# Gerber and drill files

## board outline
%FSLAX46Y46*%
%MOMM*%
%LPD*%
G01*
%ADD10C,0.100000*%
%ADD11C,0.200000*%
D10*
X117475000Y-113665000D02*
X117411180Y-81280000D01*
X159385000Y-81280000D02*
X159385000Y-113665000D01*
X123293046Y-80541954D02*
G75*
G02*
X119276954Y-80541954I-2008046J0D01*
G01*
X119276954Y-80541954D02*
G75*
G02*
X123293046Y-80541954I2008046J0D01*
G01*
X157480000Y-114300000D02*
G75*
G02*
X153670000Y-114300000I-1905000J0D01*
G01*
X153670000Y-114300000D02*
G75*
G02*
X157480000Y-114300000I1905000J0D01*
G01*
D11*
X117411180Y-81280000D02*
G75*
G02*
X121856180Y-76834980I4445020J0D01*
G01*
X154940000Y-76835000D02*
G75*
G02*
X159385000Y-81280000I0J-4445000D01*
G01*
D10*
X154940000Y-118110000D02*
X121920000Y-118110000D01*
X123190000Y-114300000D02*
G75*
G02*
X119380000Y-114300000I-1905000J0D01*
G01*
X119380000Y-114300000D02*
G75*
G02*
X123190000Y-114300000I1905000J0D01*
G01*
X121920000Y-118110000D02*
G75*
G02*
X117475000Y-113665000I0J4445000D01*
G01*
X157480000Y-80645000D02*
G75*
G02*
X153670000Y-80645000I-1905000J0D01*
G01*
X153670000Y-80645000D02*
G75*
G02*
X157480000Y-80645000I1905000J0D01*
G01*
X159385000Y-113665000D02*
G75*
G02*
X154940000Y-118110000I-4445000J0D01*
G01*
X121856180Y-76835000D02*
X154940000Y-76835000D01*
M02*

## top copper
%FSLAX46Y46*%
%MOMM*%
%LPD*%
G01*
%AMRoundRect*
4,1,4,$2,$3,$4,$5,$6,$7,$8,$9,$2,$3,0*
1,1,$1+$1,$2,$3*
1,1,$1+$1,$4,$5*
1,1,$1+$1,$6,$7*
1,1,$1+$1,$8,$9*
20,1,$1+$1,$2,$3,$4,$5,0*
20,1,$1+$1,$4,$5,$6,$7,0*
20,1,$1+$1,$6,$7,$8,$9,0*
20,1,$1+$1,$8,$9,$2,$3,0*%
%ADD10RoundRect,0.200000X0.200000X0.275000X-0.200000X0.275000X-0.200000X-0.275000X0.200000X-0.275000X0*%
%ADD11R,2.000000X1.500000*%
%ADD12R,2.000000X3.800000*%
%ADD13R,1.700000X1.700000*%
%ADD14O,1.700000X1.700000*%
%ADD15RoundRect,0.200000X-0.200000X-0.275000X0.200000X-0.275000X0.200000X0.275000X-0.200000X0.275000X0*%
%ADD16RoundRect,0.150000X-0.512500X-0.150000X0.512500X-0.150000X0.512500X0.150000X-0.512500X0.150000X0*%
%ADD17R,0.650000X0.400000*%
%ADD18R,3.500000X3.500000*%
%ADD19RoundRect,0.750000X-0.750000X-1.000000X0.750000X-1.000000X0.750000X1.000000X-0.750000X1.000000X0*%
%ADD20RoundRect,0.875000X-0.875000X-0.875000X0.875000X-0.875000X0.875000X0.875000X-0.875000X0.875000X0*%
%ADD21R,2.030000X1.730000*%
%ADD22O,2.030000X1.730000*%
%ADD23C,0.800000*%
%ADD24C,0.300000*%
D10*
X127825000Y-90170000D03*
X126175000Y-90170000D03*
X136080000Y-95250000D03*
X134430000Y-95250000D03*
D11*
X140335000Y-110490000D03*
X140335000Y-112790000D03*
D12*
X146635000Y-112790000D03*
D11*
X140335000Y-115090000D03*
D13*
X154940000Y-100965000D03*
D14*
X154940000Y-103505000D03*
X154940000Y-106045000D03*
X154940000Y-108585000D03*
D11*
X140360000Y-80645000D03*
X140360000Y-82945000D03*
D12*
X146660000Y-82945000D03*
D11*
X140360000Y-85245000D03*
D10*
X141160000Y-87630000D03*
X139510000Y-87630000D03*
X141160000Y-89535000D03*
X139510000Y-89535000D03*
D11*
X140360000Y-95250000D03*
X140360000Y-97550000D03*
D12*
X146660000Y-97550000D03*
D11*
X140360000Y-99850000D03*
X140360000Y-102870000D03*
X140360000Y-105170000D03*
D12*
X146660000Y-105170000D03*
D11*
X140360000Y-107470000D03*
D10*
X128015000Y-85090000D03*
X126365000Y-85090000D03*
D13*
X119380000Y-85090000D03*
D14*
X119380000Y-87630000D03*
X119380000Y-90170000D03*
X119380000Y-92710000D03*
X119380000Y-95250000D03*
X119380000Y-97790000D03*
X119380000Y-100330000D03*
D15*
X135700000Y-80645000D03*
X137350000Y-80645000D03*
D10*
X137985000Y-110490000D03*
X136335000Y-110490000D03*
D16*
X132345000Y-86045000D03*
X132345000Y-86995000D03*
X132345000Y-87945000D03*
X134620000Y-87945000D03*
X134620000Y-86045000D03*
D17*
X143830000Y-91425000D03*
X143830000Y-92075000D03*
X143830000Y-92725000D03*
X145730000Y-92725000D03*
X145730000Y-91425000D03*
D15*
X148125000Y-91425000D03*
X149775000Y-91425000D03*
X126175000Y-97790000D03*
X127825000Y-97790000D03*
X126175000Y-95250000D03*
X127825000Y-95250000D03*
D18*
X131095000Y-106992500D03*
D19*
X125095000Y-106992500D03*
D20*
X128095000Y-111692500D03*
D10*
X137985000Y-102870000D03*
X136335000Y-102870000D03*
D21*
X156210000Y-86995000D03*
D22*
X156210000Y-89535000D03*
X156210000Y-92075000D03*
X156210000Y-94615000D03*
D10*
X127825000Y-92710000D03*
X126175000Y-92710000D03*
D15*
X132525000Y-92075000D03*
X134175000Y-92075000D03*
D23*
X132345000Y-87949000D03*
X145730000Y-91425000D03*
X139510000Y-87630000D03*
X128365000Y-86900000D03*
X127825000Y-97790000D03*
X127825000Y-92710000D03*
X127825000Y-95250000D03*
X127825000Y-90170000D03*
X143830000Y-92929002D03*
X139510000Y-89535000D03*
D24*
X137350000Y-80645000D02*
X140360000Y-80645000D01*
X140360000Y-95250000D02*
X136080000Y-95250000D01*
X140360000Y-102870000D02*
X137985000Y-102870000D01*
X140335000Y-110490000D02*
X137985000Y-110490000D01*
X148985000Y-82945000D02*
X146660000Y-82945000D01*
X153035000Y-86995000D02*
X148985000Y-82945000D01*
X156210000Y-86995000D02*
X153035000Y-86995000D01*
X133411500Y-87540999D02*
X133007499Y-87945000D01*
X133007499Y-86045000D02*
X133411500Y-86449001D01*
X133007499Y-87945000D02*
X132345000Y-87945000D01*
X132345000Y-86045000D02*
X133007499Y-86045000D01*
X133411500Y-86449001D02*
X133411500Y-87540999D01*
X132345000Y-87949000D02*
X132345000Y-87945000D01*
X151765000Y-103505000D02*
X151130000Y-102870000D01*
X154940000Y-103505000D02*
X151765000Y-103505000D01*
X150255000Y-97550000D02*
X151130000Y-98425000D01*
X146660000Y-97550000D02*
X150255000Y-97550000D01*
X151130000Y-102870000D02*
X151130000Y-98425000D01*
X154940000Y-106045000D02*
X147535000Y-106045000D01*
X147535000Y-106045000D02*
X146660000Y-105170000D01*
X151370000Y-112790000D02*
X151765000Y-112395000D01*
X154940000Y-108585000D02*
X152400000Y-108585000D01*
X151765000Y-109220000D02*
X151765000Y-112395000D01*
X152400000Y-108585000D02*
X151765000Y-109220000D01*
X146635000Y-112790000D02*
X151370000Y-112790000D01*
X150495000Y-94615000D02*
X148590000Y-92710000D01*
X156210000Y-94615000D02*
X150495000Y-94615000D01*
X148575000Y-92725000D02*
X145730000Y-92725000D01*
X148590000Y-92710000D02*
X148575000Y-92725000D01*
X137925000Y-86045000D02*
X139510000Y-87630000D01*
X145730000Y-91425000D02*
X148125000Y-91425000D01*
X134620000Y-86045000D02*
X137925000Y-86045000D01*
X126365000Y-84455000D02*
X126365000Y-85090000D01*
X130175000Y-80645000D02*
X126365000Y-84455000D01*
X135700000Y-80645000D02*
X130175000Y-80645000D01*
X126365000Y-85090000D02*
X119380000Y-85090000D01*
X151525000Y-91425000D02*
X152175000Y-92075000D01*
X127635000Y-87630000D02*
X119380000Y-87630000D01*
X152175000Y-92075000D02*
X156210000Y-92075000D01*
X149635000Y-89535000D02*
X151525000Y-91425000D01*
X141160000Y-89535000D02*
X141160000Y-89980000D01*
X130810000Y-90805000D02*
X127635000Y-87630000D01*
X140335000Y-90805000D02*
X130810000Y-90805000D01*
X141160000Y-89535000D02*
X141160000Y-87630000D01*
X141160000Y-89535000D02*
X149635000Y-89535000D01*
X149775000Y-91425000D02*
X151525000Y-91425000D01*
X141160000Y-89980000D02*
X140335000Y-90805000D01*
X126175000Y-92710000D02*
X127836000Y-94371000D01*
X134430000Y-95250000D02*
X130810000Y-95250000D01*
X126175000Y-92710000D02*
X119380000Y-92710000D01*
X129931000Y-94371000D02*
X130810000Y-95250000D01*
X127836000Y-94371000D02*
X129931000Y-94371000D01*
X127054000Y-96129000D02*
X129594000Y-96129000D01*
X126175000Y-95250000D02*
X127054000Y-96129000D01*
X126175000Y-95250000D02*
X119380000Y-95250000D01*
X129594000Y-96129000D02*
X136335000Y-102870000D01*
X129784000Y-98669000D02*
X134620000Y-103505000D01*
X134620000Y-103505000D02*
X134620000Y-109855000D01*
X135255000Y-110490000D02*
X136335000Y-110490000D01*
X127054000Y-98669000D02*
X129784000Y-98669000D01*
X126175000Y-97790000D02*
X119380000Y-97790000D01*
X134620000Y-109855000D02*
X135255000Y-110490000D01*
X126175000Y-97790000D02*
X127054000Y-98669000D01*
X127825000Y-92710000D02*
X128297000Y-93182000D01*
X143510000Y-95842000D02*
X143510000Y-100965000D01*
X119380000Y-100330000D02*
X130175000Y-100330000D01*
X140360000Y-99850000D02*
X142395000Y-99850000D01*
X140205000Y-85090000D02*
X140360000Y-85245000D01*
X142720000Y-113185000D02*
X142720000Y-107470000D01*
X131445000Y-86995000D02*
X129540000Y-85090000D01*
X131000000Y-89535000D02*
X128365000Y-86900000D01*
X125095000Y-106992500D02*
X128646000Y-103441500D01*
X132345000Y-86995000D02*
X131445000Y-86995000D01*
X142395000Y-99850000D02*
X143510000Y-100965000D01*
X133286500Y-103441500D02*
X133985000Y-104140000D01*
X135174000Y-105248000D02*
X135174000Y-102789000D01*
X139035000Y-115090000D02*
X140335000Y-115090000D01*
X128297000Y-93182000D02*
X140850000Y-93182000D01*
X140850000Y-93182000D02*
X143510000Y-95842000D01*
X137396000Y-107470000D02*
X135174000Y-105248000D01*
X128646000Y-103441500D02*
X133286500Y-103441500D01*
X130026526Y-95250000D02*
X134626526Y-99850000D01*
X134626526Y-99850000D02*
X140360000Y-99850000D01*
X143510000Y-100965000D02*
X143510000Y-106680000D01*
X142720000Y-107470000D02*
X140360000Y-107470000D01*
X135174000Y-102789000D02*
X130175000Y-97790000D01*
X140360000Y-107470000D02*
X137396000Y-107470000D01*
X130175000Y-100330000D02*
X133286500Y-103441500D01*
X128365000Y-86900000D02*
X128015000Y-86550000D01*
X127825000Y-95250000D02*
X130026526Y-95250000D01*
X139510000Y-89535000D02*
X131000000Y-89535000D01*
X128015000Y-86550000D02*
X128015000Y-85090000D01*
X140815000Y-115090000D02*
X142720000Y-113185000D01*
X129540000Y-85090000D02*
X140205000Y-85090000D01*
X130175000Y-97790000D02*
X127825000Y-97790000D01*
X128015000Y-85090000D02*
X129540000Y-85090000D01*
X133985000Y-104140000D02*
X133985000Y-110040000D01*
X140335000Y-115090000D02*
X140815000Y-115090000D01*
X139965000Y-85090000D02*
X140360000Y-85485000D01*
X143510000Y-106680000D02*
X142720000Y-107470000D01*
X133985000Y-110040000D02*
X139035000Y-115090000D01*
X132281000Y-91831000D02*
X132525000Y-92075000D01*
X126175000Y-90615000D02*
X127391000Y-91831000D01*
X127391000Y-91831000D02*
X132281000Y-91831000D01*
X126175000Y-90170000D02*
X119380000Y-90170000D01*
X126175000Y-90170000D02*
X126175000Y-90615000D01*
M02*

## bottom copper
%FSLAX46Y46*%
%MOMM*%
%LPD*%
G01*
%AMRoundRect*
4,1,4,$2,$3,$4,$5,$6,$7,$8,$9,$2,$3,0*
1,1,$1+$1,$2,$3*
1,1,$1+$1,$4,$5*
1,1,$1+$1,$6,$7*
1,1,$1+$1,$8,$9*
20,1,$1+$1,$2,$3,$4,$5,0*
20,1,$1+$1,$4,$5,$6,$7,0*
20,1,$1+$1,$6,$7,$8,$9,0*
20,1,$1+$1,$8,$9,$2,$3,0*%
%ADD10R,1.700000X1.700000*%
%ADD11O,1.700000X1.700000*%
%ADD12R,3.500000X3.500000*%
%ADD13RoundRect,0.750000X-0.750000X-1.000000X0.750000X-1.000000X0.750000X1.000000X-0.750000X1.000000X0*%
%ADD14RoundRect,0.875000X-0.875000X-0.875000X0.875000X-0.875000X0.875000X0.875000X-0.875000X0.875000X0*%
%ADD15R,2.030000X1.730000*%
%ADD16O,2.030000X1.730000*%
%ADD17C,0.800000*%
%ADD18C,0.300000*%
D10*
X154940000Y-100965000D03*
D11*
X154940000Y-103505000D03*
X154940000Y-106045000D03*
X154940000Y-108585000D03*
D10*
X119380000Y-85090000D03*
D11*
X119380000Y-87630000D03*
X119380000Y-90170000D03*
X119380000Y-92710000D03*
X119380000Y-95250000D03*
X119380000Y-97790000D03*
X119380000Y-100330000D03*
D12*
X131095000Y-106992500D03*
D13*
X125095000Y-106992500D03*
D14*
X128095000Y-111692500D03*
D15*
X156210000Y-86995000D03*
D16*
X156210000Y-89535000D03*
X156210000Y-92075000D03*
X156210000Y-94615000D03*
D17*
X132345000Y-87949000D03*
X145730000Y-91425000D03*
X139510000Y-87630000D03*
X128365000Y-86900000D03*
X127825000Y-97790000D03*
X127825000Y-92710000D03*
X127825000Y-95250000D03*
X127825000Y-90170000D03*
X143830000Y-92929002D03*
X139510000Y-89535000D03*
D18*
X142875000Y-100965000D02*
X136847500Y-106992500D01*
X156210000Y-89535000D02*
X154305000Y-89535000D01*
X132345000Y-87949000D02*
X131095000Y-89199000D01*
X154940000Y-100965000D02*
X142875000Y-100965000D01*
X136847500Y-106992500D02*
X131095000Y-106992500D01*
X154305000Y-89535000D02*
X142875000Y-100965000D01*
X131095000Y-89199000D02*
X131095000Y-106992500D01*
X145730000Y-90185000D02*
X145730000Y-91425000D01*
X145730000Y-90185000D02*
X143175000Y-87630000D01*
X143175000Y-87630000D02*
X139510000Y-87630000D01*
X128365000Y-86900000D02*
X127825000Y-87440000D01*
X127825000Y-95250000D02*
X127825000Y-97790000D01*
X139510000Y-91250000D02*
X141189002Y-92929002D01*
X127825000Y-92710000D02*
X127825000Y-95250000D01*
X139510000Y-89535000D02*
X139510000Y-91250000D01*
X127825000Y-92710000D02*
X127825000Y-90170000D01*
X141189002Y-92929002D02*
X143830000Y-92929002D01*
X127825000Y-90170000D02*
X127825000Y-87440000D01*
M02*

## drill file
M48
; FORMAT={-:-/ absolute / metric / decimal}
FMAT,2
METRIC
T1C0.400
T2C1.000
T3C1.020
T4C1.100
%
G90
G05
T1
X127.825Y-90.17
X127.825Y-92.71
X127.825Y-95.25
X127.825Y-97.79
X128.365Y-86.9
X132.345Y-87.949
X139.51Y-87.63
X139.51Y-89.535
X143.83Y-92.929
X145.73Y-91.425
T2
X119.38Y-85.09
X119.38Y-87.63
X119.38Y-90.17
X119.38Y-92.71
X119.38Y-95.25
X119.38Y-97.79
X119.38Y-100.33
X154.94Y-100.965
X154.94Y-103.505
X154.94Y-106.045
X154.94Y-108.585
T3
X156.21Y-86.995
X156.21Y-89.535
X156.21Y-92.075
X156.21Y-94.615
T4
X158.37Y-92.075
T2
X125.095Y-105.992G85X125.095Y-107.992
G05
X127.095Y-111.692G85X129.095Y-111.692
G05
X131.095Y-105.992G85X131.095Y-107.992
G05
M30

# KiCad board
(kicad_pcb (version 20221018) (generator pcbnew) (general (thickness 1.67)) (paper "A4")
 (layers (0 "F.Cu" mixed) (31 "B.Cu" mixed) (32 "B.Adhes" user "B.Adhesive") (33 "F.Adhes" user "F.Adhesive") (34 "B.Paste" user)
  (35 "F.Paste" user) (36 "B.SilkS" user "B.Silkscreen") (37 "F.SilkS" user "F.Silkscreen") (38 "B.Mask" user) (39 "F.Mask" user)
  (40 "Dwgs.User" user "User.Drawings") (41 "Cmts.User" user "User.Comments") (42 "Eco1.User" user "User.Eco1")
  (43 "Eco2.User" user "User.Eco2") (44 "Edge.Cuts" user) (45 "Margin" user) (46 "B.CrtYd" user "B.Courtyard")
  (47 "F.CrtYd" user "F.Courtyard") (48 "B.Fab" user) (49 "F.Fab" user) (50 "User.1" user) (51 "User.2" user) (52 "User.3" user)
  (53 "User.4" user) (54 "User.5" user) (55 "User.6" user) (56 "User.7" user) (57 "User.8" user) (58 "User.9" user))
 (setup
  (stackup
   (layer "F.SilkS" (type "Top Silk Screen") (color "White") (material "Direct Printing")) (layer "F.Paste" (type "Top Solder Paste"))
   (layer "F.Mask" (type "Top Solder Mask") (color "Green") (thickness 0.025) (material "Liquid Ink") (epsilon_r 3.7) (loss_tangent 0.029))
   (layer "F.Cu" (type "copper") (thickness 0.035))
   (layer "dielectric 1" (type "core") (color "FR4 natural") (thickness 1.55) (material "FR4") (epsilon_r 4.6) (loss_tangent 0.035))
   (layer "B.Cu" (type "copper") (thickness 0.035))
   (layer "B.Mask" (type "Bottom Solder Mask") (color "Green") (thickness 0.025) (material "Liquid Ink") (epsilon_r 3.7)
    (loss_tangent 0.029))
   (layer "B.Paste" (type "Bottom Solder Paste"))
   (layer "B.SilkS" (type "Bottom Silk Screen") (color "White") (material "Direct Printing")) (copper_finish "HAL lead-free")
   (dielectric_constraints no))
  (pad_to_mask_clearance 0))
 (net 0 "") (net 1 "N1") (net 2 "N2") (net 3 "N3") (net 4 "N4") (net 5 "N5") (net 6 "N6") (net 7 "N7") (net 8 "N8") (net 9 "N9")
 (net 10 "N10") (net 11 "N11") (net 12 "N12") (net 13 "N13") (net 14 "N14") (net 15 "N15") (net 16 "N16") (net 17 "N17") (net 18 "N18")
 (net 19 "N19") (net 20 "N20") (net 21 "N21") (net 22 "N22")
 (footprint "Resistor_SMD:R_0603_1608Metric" (layer "F.Cu") (at 127 90.17 180)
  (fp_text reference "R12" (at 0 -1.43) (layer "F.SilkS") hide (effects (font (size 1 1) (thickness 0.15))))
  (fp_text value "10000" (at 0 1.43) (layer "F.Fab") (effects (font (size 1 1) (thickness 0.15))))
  (pad "1" smd roundrect (at -0.825 0 180) (size 0.8 0.95) (layers "F.Cu" "F.Paste" "F.Mask") (roundrect_rratio 0.25) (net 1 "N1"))
  (pad "2" smd roundrect (at 0.825 0 180) (size 0.8 0.95) (layers "F.Cu" "F.Paste" "F.Mask") (roundrect_rratio 0.25) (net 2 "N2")))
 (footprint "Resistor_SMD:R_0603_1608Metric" (layer "F.Cu") (at 135.255 95.25 180)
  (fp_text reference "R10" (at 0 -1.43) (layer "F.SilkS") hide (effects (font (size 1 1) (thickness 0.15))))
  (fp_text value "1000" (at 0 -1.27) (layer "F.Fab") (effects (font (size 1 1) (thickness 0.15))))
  (pad "1" smd roundrect (at -0.825 0 180) (size 0.8 0.95) (layers "F.Cu" "F.Paste" "F.Mask") (roundrect_rratio 0.25) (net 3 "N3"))
  (pad "2" smd roundrect (at 0.825 0 180) (size 0.8 0.95) (layers "F.Cu" "F.Paste" "F.Mask") (roundrect_rratio 0.25) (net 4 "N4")))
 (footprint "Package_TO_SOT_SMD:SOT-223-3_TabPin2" (layer "F.Cu") (at 143.485 112.79)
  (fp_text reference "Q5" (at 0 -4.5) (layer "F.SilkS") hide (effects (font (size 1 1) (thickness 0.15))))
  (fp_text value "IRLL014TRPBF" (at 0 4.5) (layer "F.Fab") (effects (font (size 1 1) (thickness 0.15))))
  (pad "1" smd rect (at -3.15 -2.3) (size 2 1.5) (layers "F.Cu" "F.Paste" "F.Mask") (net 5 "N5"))
  (pad "2" smd rect (at -3.15 0) (size 2 1.5) (layers "F.Cu" "F.Paste" "F.Mask") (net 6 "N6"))
  (pad "2" smd rect (at 3.15 0) (size 2 3.8) (layers "F.Cu" "F.Paste" "F.Mask") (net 6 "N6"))
  (pad "3" smd rect (at -3.15 2.3) (size 2 1.5) (layers "F.Cu" "F.Paste" "F.Mask") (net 1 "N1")))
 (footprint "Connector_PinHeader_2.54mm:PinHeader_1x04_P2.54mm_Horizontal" (layer "F.Cu") (at 154.94 100.965)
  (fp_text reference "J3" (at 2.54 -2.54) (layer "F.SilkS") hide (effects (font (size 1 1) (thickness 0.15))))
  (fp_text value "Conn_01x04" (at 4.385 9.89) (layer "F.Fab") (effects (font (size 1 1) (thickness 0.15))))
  (pad "1" thru_hole rect (at 0 0) (size 1.7 1.7) (drill 1) (layers "*.Cu" "*.Mask") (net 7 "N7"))
  (pad "2" thru_hole oval (at 0 2.54) (size 1.7 1.7) (drill 1) (layers "*.Cu" "*.Mask") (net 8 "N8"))
  (pad "3" thru_hole oval (at 0 5.08) (size 1.7 1.7) (drill 1) (layers "*.Cu" "*.Mask") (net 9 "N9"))
  (pad "4" thru_hole oval (at 0 7.62) (size 1.7 1.7) (drill 1) (layers "*.Cu" "*.Mask") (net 6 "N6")))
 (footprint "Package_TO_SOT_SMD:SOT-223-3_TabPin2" (layer "F.Cu") (at 143.51 82.945)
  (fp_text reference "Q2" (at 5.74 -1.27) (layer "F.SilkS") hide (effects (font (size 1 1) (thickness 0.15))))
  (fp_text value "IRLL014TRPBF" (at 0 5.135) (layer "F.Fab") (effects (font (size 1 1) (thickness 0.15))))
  (pad "1" smd rect (at -3.15 -2.3) (size 2 1.5) (layers "F.Cu" "F.Paste" "F.Mask") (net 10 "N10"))
  (pad "2" smd rect (at -3.15 0) (size 2 1.5) (layers "F.Cu" "F.Paste" "F.Mask") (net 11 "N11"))
  (pad "2" smd rect (at 3.15 0) (size 2 3.8) (layers "F.Cu" "F.Paste" "F.Mask") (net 11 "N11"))
  (pad "3" smd rect (at -3.15 2.3) (size 2 1.5) (layers "F.Cu" "F.Paste" "F.Mask") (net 1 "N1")))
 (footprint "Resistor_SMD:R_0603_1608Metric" (layer "F.Cu") (at 140.335 87.63 180)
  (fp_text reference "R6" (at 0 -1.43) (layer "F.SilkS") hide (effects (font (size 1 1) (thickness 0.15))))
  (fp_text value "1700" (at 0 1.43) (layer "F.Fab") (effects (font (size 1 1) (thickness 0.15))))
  (pad "1" smd roundrect (at -0.825 0 180) (size 0.8 0.95) (layers "F.Cu" "F.Paste" "F.Mask") (roundrect_rratio 0.25) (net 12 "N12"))
  (pad "2" smd roundrect (at 0.825 0 180) (size 0.8 0.95) (layers "F.Cu" "F.Paste" "F.Mask") (roundrect_rratio 0.25) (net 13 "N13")))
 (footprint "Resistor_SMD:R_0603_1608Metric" (layer "F.Cu") (at 140.335 89.535 180)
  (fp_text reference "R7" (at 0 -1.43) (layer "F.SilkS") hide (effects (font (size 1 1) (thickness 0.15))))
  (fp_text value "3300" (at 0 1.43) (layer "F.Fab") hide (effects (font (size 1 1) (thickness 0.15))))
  (pad "1" smd roundrect (at -0.825 0 180) (size 0.8 0.95) (layers "F.Cu" "F.Paste" "F.Mask") (roundrect_rratio 0.25) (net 12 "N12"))
  (pad "2" smd roundrect (at 0.825 0 180) (size 0.8 0.95) (layers "F.Cu" "F.Paste" "F.Mask") (roundrect_rratio 0.25) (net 1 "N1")))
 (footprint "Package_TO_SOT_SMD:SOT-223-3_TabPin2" (layer "F.Cu") (at 143.51 97.55)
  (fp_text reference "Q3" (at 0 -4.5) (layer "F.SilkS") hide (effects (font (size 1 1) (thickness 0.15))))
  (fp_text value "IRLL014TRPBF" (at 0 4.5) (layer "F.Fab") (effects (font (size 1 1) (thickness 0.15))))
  (pad "1" smd rect (at -3.15 -2.3) (size 2 1.5) (layers "F.Cu" "F.Paste" "F.Mask") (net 3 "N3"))
  (pad "2" smd rect (at -3.15 0) (size 2 1.5) (layers "F.Cu" "F.Paste" "F.Mask") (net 8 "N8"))
  (pad "2" smd rect (at 3.15 0) (size 2 3.8) (layers "F.Cu" "F.Paste" "F.Mask") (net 8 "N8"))
  (pad "3" smd rect (at -3.15 2.3) (size 2 1.5) (layers "F.Cu" "F.Paste" "F.Mask") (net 1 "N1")))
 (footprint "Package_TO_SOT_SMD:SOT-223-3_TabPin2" (layer "F.Cu") (at 143.51 105.17)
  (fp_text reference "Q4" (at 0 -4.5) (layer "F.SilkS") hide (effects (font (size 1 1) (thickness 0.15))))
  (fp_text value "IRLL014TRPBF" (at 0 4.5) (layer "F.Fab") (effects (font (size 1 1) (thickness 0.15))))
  (pad "1" smd rect (at -3.15 -2.3) (size 2 1.5) (layers "F.Cu" "F.Paste" "F.Mask") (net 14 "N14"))
  (pad "2" smd rect (at -3.15 0) (size 2 1.5) (layers "F.Cu" "F.Paste" "F.Mask") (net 9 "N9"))
  (pad "2" smd rect (at 3.15 0) (size 2 3.8) (layers "F.Cu" "F.Paste" "F.Mask") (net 9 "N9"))
  (pad "3" smd rect (at -3.15 2.3) (size 2 1.5) (layers "F.Cu" "F.Paste" "F.Mask") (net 1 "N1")))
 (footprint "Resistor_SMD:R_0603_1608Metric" (layer "F.Cu") (at 127.19 85.09 180)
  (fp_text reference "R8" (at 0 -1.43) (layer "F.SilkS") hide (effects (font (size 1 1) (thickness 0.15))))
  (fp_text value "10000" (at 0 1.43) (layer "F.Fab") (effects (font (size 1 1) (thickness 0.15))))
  (pad "1" smd roundrect (at -0.825 0 180) (size 0.8 0.95) (layers "F.Cu" "F.Paste" "F.Mask") (roundrect_rratio 0.25) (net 1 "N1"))
  (pad "2" smd roundrect (at 0.825 0 180) (size 0.8 0.95) (layers "F.Cu" "F.Paste" "F.Mask") (roundrect_rratio 0.25) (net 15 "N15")))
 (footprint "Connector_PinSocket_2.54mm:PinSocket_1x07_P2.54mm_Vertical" (layer "F.Cu") (at 119.38 85.09)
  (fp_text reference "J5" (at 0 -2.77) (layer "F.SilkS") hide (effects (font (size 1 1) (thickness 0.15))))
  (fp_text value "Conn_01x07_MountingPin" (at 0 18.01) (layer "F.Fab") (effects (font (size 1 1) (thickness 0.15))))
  (pad "1" thru_hole rect (at 0 0) (size 1.7 1.7) (drill 1) (layers "*.Cu" "*.Mask") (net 15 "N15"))
  (pad "2" thru_hole oval (at 0 2.54) (size 1.7 1.7) (drill 1) (layers "*.Cu" "*.Mask") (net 12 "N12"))
  (pad "3" thru_hole oval (at 0 5.08) (size 1.7 1.7) (drill 1) (layers "*.Cu" "*.Mask") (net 2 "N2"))
  (pad "4" thru_hole oval (at 0 7.62) (size 1.7 1.7) (drill 1) (layers "*.Cu" "*.Mask") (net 4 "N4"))
  (pad "5" thru_hole oval (at 0 10.16) (size 1.7 1.7) (drill 1) (layers "*.Cu" "*.Mask") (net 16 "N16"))
  (pad "6" thru_hole oval (at 0 12.7) (size 1.7 1.7) (drill 1) (layers "*.Cu" "*.Mask") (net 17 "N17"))
  (pad "7" thru_hole oval (at 0 15.24) (size 1.7 1.7) (drill 1) (layers "*.Cu" "*.Mask") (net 1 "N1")))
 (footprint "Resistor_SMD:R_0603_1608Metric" (layer "F.Cu") (at 136.525 80.645)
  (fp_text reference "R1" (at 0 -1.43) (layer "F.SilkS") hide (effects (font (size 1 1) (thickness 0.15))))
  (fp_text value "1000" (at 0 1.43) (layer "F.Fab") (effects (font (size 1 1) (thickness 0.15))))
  (pad "1" smd roundrect (at -0.825 0) (size 0.8 0.95) (layers "F.Cu" "F.Paste" "F.Mask") (roundrect_rratio 0.25) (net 15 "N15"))
  (pad "2" smd roundrect (at 0.825 0) (size 0.8 0.95) (layers "F.Cu" "F.Paste" "F.Mask") (roundrect_rratio 0.25) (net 10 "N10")))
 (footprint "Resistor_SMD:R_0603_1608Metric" (layer "F.Cu") (at 137.16 110.49 180)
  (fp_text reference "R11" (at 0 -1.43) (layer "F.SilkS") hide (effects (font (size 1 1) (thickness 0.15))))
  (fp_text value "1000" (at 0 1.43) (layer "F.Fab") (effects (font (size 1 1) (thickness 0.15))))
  (pad "1" smd roundrect (at -0.825 0 180) (size 0.8 0.95) (layers "F.Cu" "F.Paste" "F.Mask") (roundrect_rratio 0.25) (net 5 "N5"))
  (pad "2" smd roundrect (at 0.825 0 180) (size 0.8 0.95) (layers "F.Cu" "F.Paste" "F.Mask") (roundrect_rratio 0.25) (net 17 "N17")))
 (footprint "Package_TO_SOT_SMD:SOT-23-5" (layer "F.Cu") (at 133.4825 86.995)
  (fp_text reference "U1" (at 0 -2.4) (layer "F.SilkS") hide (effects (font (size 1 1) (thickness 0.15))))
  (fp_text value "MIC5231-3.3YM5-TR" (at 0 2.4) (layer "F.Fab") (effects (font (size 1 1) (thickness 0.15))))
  (pad "1" smd roundrect (at -1.1375 -0.95) (size 1.325 0.6) (layers "F.Cu" "F.Paste" "F.Mask") (roundrect_rratio 0.25) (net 7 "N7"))
  (pad "2" smd roundrect (at -1.1375 0) (size 1.325 0.6) (layers "F.Cu" "F.Paste" "F.Mask") (roundrect_rratio 0.25) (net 1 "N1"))
  (pad "3" smd roundrect (at -1.1375 0.95) (size 1.325 0.6) (layers "F.Cu" "F.Paste" "F.Mask") (roundrect_rratio 0.25) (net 7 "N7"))
  (pad "4" smd roundrect (at 1.1375 0.95) (size 1.325 0.6) (layers "F.Cu" "F.Paste" "F.Mask") (roundrect_rratio 0.25) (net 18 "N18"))
  (pad "5" smd roundrect (at 1.1375 -0.95) (size 1.325 0.6) (layers "F.Cu" "F.Paste" "F.Mask") (roundrect_rratio 0.25) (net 13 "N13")))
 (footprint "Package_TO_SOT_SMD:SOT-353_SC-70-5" (layer "F.Cu") (at 144.78 92.075)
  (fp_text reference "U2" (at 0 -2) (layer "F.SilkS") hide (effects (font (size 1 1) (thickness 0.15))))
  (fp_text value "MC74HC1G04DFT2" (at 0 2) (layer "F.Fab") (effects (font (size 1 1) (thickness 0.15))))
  (pad "1" smd rect (at -0.95 -0.65) (size 0.65 0.4) (layers "F.Cu" "F.Paste" "F.Mask") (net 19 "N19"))
  (pad "2" smd rect (at -0.95 0) (size 0.65 0.4) (layers "F.Cu" "F.Paste" "F.Mask") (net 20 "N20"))
  (pad "3" smd rect (at -0.95 0.65) (size 0.65 0.4) (layers "F.Cu" "F.Paste" "F.Mask") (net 1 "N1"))
  (pad "4" smd rect (at 0.95 0.65) (size 0.65 0.4) (layers "F.Cu" "F.Paste" "F.Mask") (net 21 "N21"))
  (pad "5" smd rect (at 0.95 -0.65) (size 0.65 0.4) (layers "F.Cu" "F.Paste" "F.Mask") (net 13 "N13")))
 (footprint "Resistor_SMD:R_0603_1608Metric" (layer "F.Cu") (at 148.95 91.425)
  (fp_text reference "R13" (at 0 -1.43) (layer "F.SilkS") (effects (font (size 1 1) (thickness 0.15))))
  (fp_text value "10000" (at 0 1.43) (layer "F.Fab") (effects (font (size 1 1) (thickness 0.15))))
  (pad "1" smd roundrect (at -0.825 0) (size 0.8 0.95) (layers "F.Cu" "F.Paste" "F.Mask") (roundrect_rratio 0.25) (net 13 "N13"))
  (pad "2" smd roundrect (at 0.825 0) (size 0.8 0.95) (layers "F.Cu" "F.Paste" "F.Mask") (roundrect_rratio 0.25) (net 12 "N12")))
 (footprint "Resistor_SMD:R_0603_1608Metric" (layer "F.Cu") (at 127 97.79)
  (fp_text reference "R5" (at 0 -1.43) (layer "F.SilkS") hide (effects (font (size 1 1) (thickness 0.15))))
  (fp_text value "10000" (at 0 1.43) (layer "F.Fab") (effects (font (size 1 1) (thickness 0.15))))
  (pad "1" smd roundrect (at -0.825 0) (size 0.8 0.95) (layers "F.Cu" "F.Paste" "F.Mask") (roundrect_rratio 0.25) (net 17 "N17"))
  (pad "2" smd roundrect (at 0.825 0) (size 0.8 0.95) (layers "F.Cu" "F.Paste" "F.Mask") (roundrect_rratio 0.25) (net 1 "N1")))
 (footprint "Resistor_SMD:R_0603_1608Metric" (layer "F.Cu") (at 127 95.25)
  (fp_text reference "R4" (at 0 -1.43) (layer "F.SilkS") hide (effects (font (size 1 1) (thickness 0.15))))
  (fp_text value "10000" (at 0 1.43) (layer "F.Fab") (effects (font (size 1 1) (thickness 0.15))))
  (pad "1" smd roundrect (at -0.825 0) (size 0.8 0.95) (layers "F.Cu" "F.Paste" "F.Mask") (roundrect_rratio 0.25) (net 16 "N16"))
  (pad "2" smd roundrect (at 0.825 0) (size 0.8 0.95) (layers "F.Cu" "F.Paste" "F.Mask") (roundrect_rratio 0.25) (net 1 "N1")))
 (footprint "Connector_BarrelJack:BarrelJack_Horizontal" (layer "F.Cu") (at 131.095 106.9925)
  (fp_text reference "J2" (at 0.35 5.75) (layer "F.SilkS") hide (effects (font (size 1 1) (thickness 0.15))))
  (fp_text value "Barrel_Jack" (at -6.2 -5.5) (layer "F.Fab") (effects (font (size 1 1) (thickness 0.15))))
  (pad "1" thru_hole rect (at 0 0) (size 3.5 3.5) (drill oval 1 3) (layers "*.Cu" "*.Mask") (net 7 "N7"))
  (pad "2" thru_hole roundrect (at -6 0) (size 3 3.5) (drill oval 1 3) (layers "*.Cu" "*.Mask") (roundrect_rratio 0.25) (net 1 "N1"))
  (pad "3" thru_hole roundrect (at -3 4.7) (size 3.5 3.5) (drill oval 3 1) (layers "*.Cu" "*.Mask") (roundrect_rratio 0.25)))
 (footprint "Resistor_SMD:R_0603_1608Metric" (layer "F.Cu") (at 137.16 102.87 180)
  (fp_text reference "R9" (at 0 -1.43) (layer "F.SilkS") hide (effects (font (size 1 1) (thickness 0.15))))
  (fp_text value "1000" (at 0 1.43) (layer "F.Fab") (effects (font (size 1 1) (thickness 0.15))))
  (pad "1" smd roundrect (at -0.825 0 180) (size 0.8 0.95) (layers "F.Cu" "F.Paste" "F.Mask") (roundrect_rratio 0.25) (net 14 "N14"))
  (pad "2" smd roundrect (at 0.825 0 180) (size 0.8 0.95) (layers "F.Cu" "F.Paste" "F.Mask") (roundrect_rratio 0.25) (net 16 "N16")))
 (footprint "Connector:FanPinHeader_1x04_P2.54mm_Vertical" (layer "F.Cu") (at 156.21 86.995 -90)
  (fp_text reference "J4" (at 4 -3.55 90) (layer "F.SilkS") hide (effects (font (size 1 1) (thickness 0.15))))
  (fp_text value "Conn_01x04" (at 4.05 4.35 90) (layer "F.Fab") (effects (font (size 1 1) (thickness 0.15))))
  (pad "" np_thru_hole circle (at 5.08 -2.16) (size 1.1 1.1) (drill 1.1) (layers "*.Cu" "*.Mask"))
  (pad "1" thru_hole rect (at 0 0) (size 2.03 1.73) (drill 1.02) (layers "*.Cu" "*.Mask") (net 11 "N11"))
  (pad "2" thru_hole oval (at 2.54 0) (size 2.03 1.73) (drill 1.02) (layers "*.Cu" "*.Mask") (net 7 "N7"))
  (pad "3" thru_hole oval (at 5.08 0) (size 2.03 1.73) (drill 1.02) (layers "*.Cu" "*.Mask") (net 12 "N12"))
  (pad "4" thru_hole oval (at 7.62 0) (size 2.03 1.73) (drill 1.02) (layers "*.Cu" "*.Mask") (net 21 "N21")))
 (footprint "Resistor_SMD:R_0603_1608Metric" (layer "F.Cu") (at 127 92.71 180)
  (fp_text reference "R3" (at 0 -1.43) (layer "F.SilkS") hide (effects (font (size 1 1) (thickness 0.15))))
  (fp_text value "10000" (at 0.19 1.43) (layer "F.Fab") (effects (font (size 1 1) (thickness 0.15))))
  (pad "1" smd roundrect (at -0.825 0 180) (size 0.8 0.95) (layers "F.Cu" "F.Paste" "F.Mask") (roundrect_rratio 0.25) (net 1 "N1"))
  (pad "2" smd roundrect (at 0.825 0 180) (size 0.8 0.95) (layers "F.Cu" "F.Paste" "F.Mask") (roundrect_rratio 0.25) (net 4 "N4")))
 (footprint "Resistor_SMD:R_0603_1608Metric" (layer "F.Cu") (at 133.35 92.075)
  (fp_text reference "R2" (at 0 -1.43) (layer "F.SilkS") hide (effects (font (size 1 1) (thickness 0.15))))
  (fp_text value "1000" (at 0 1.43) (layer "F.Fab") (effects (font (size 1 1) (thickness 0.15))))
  (pad "1" smd roundrect (at -0.825 0) (size 0.8 0.95) (layers "F.Cu" "F.Paste" "F.Mask") (roundrect_rratio 0.25) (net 2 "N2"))
  (pad "2" smd roundrect (at 0.825 0) (size 0.8 0.95) (layers "F.Cu" "F.Paste" "F.Mask") (roundrect_rratio 0.25) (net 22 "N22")))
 (gr_line (start 117.475 113.665) (end 117.41118 81.28) (stroke (width 0.1) (type default)) (layer "Edge.Cuts"))
 (gr_line (start 159.385 81.28) (end 159.385 113.665) (stroke (width 0.1) (type default)) (layer "Edge.Cuts"))
 (gr_circle (center 121.285 80.541954) (end 123.19 81.176954) (stroke (width 0.1) (type default)) (fill none) (layer "Edge.Cuts"))
 (gr_circle (center 155.575 114.3) (end 157.48 114.3) (stroke (width 0.1) (type default)) (fill none) (layer "Edge.Cuts"))
 (gr_arc (start 117.41118 81.28) (mid 118.71309 78.13691) (end 121.85618 76.835) (stroke (width 0.2) (type default)) (layer "Edge.Cuts"))
 (gr_arc (start 154.94 76.835) (mid 158.08309 78.13691) (end 159.385 81.28) (stroke (width 0.2) (type default)) (layer "Edge.Cuts"))
 (gr_line (start 154.94 118.11) (end 121.92 118.11) (stroke (width 0.1) (type default)) (layer "Edge.Cuts"))
 (gr_circle (center 121.285 114.3) (end 123.19 114.3) (stroke (width 0.1) (type default)) (fill none) (layer "Edge.Cuts"))
 (gr_arc (start 121.92 118.11) (mid 118.77691 116.80809) (end 117.475 113.665) (stroke (width 0.1) (type default)) (layer "Edge.Cuts"))
 (gr_circle (center 155.575 80.645) (end 157.48 80.645) (stroke (width 0.1) (type default)) (fill none) (layer "Edge.Cuts"))
 (gr_arc (start 159.385 113.665) (mid 158.08309 116.80809) (end 154.94 118.11) (stroke (width 0.1) (type default)) (layer "Edge.Cuts"))
 (gr_line (start 121.85618 76.835) (end 154.94 76.835) (stroke (width 0.1) (type default)) (layer "Edge.Cuts"))
 (segment (start 137.35 80.645) (end 140.36 80.645) (width 0.3) (layer "F.Cu") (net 10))
 (segment (start 140.36 95.25) (end 136.08 95.25) (width 0.3) (layer "F.Cu") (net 3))
 (segment (start 140.36 102.87) (end 137.985 102.87) (width 0.3) (layer "F.Cu") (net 14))
 (segment (start 140.335 110.49) (end 137.985 110.49) (width 0.3) (layer "F.Cu") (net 5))
 (segment (start 148.985 82.945) (end 146.66 82.945) (width 0.3) (layer "F.Cu") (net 11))
 (segment (start 153.035 86.995) (end 148.985 82.945) (width 0.3) (layer "F.Cu") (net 11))
 (segment (start 156.21 86.995) (end 153.035 86.995) (width 0.3) (layer "F.Cu") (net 11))
 (segment (start 133.4115 87.540999) (end 133.007499 87.945) (width 0.3) (layer "F.Cu") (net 7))
 (segment (start 133.007499 86.045) (end 133.4115 86.449001) (width 0.3) (layer "F.Cu") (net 7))
 (segment (start 133.007499 87.945) (end 132.345 87.945) (width 0.3) (layer "F.Cu") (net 7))
 (segment (start 132.345 86.045) (end 133.007499 86.045) (width 0.3) (layer "F.Cu") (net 7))
 (segment (start 133.4115 86.449001) (end 133.4115 87.540999) (width 0.3) (layer "F.Cu") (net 7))
 (segment (start 132.345 87.949) (end 132.345 87.945) (width 0.3) (layer "F.Cu") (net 7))
 (via (at 132.345 87.949) (size 0.8) (drill 0.4) (layers "F.Cu" "B.Cu") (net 7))
 (segment (start 142.875 100.965) (end 136.8475 106.9925) (width 0.3) (layer "B.Cu") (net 7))
 (segment (start 156.21 89.535) (end 154.305 89.535) (width 0.3) (layer "B.Cu") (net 7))
 (segment (start 132.345 87.949) (end 131.095 89.199) (width 0.3) (layer "B.Cu") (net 7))
 (segment (start 154.94 100.965) (end 142.875 100.965) (width 0.3) (layer "B.Cu") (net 7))
 (segment (start 136.8475 106.9925) (end 131.095 106.9925) (width 0.3) (layer "B.Cu") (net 7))
 (segment (start 154.305 89.535) (end 142.875 100.965) (width 0.3) (layer "B.Cu") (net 7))
 (segment (start 131.095 89.199) (end 131.095 106.9925) (width 0.3) (layer "B.Cu") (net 7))
 (segment (start 151.765 103.505) (end 151.13 102.87) (width 0.3) (layer "F.Cu") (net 8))
 (segment (start 154.94 103.505) (end 151.765 103.505) (width 0.3) (layer "F.Cu") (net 8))
 (segment (start 150.255 97.55) (end 151.13 98.425) (width 0.3) (layer "F.Cu") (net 8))
 (segment (start 146.66 97.55) (end 150.255 97.55) (width 0.3) (layer "F.Cu") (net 8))
 (segment (start 151.13 102.87) (end 151.13 98.425) (width 0.3) (layer "F.Cu") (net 8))
 (segment (start 154.94 106.045) (end 147.535 106.045) (width 0.3) (layer "F.Cu") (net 9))
 (segment (start 147.535 106.045) (end 146.66 105.17) (width 0.3) (layer "F.Cu") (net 9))
 (segment (start 151.37 112.79) (end 151.765 112.395) (width 0.3) (layer "F.Cu") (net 6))
 (segment (start 154.94 108.585) (end 152.4 108.585) (width 0.3) (layer "F.Cu") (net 6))
 (segment (start 151.765 109.22) (end 151.765 112.395) (width 0.3) (layer "F.Cu") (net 6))
 (segment (start 152.4 108.585) (end 151.765 109.22) (width 0.3) (layer "F.Cu") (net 6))
 (segment (start 146.635 112.79) (end 151.37 112.79) (width 0.3) (layer "F.Cu") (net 6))
 (segment (start 150.495 94.615) (end 148.59 92.71) (width 0.3) (layer "F.Cu") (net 21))
 (segment (start 156.21 94.615) (end 150.495 94.615) (width 0.3) (layer "F.Cu") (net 21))
 (segment (start 148.575 92.725) (end 145.73 92.725) (width 0.3) (layer "F.Cu") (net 21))
 (segment (start 148.59 92.71) (end 148.575 92.725) (width 0.3) (layer "F.Cu") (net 21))
 (segment (start 137.925 86.045) (end 139.51 87.63) (width 0.3) (layer "F.Cu") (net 13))
 (segment (start 145.73 91.425) (end 148.125 91.425) (width 0.3) (layer "F.Cu") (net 13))
 (segment (start 134.62 86.045) (end 137.925 86.045) (width 0.3) (layer "F.Cu") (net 13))
 (via (at 145.73 91.425) (size 0.8) (drill 0.4) (layers "F.Cu" "B.Cu") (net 13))
 (via (at 139.51 87.63) (size 0.8) (drill 0.4) (layers "F.Cu" "B.Cu") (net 13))
 (segment (start 145.73 90.185) (end 145.73 91.425) (width 0.3) (layer "B.Cu") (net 13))
 (segment (start 145.73 90.185) (end 143.175 87.63) (width 0.3) (layer "B.Cu") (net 13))
 (segment (start 143.175 87.63) (end 139.51 87.63) (width 0.3) (layer "B.Cu") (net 13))
 (segment (start 126.365 84.455) (end 126.365 85.09) (width 0.3) (layer "F.Cu") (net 15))
 (segment (start 130.175 80.645) (end 126.365 84.455) (width 0.3) (layer "F.Cu") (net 15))
 (segment (start 135.7 80.645) (end 130.175 80.645) (width 0.3) (layer "F.Cu") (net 15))
 (segment (start 126.365 85.09) (end 119.38 85.09) (width 0.3) (layer "F.Cu") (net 15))
 (segment (start 151.525 91.425) (end 152.175 92.075) (width 0.3) (layer "F.Cu") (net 12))
 (segment (start 127.635 87.63) (end 119.38 87.63) (width 0.3) (layer "F.Cu") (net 12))
 (segment (start 152.175 92.075) (end 156.21 92.075) (width 0.3) (layer "F.Cu") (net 12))
 (segment (start 149.635 89.535) (end 151.525 91.425) (width 0.3) (layer "F.Cu") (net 12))
 (segment (start 141.16 89.535) (end 141.16 89.98) (width 0.3) (layer "F.Cu") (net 12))
 (segment (start 130.81 90.805) (end 127.635 87.63) (width 0.3) (layer "F.Cu") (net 12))
 (segment (start 140.335 90.805) (end 130.81 90.805) (width 0.3) (layer "F.Cu") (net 12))
 (segment (start 141.16 89.535) (end 141.16 87.63) (width 0.3) (layer "F.Cu") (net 12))
 (segment (start 141.16 89.535) (end 149.635 89.535) (width 0.3) (layer "F.Cu") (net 12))
 (segment (start 149.775 91.425) (end 151.525 91.425) (width 0.3) (layer "F.Cu") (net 12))
 (segment (start 141.16 89.98) (end 140.335 90.805) (width 0.3) (layer "F.Cu") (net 12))
 (segment (start 126.175 92.71) (end 127.836 94.371) (width 0.3) (layer "F.Cu") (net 4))
 (segment (start 134.43 95.25) (end 130.81 95.25) (width 0.3) (layer "F.Cu") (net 4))
 (segment (start 126.175 92.71) (end 119.38 92.71) (width 0.3) (layer "F.Cu") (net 4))
 (segment (start 129.931 94.371) (end 130.81 95.25) (width 0.3) (layer "F.Cu") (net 4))
 (segment (start 127.836 94.371) (end 129.931 94.371) (width 0.3) (layer "F.Cu") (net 4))
 (segment (start 127.054 96.129) (end 129.594 96.129) (width 0.3) (layer "F.Cu") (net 16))
 (segment (start 126.175 95.25) (end 127.054 96.129) (width 0.3) (layer "F.Cu") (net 16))
 (segment (start 126.175 95.25) (end 119.38 95.25) (width 0.3) (layer "F.Cu") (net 16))
 (segment (start 129.594 96.129) (end 136.335 102.87) (width 0.3) (layer "F.Cu") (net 16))
 (segment (start 129.784 98.669) (end 134.62 103.505) (width 0.3) (layer "F.Cu") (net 17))
 (segment (start 134.62 103.505) (end 134.62 109.855) (width 0.3) (layer "F.Cu") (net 17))
 (segment (start 135.255 110.49) (end 136.335 110.49) (width 0.3) (layer "F.Cu") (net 17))
 (segment (start 127.054 98.669) (end 129.784 98.669) (width 0.3) (layer "F.Cu") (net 17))
 (segment (start 126.175 97.79) (end 119.38 97.79) (width 0.3) (layer "F.Cu") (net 17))
 (segment (start 134.62 109.855) (end 135.255 110.49) (width 0.3) (layer "F.Cu") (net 17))
 (segment (start 126.175 97.79) (end 127.054 98.669) (width 0.3) (layer "F.Cu") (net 17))
 (segment (start 127.825 92.71) (end 128.297 93.182) (width 0.3) (layer "F.Cu") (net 1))
 (segment (start 143.51 95.842) (end 143.51 100.965) (width 0.3) (layer "F.Cu") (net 1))
 (segment (start 119.38 100.33) (end 130.175 100.33) (width 0.3) (layer "F.Cu") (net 1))
 (segment (start 140.36 99.85) (end 142.395 99.85) (width 0.3) (layer "F.Cu") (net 1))
 (segment (start 140.205 85.09) (end 140.36 85.245) (width 0.3) (layer "F.Cu") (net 1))
 (segment (start 142.72 113.185) (end 142.72 107.47) (width 0.3) (layer "F.Cu") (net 1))
 (segment (start 131.445 86.995) (end 129.54 85.09) (width 0.3) (layer "F.Cu") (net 1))
 (segment (start 131 89.535) (end 128.365 86.9) (width 0.3) (layer "F.Cu") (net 1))
 (segment (start 125.095 106.9925) (end 128.646 103.4415) (width 0.3) (layer "F.Cu") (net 1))
 (segment (start 132.345 86.995) (end 131.445 86.995) (width 0.3) (layer "F.Cu") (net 1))
 (segment (start 142.395 99.85) (end 143.51 100.965) (width 0.3) (layer "F.Cu") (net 1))
 (segment (start 133.2865 103.4415) (end 133.985 104.14) (width 0.3) (layer "F.Cu") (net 1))
 (segment (start 135.174 105.248) (end 135.174 102.789) (width 0.3) (layer "F.Cu") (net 1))
 (segment (start 139.035 115.09) (end 140.335 115.09) (width 0.3) (layer "F.Cu") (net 1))
 (segment (start 128.297 93.182) (end 140.85 93.182) (width 0.3) (layer "F.Cu") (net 1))
 (segment (start 140.85 93.182) (end 143.51 95.842) (width 0.3) (layer "F.Cu") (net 1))
 (segment (start 137.396 107.47) (end 135.174 105.248) (width 0.3) (layer "F.Cu") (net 1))
 (segment (start 128.646 103.4415) (end 133.2865 103.4415) (width 0.3) (layer "F.Cu") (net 1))
 (segment (start 130.026526 95.25) (end 134.626526 99.85) (width 0.3) (layer "F.Cu") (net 1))
 (segment (start 134.626526 99.85) (end 140.36 99.85) (width 0.3) (layer "F.Cu") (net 1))
 (segment (start 143.51 100.965) (end 143.51 106.68) (width 0.3) (layer "F.Cu") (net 1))
 (segment (start 142.72 107.47) (end 140.36 107.47) (width 0.3) (layer "F.Cu") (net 1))
 (segment (start 135.174 102.789) (end 130.175 97.79) (width 0.3) (layer "F.Cu") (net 1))
 (segment (start 140.36 107.47) (end 137.396 107.47) (width 0.3) (layer "F.Cu") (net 1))
 (segment (start 130.175 100.33) (end 133.2865 103.4415) (width 0.3) (layer "F.Cu") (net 1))
 (segment (start 128.365 86.9) (end 128.015 86.55) (width 0.3) (layer "F.Cu") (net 1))
 (segment (start 127.825 95.25) (end 130.026526 95.25) (width 0.3) (layer "F.Cu") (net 1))
 (segment (start 139.51 89.535) (end 131 89.535) (width 0.3) (layer "F.Cu") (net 1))
 (segment (start 128.015 86.55) (end 128.015 85.09) (width 0.3) (layer "F.Cu") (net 1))
 (segment (start 140.815 115.09) (end 142.72 113.185) (width 0.3) (layer "F.Cu") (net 1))
 (segment (start 129.54 85.09) (end 140.205 85.09) (width 0.3) (layer "F.Cu") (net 1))
 (segment (start 130.175 97.79) (end 127.825 97.79) (width 0.3) (layer "F.Cu") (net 1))
 (segment (start 128.015 85.09) (end 129.54 85.09) (width 0.3) (layer "F.Cu") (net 1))
 (segment (start 133.985 104.14) (end 133.985 110.04) (width 0.3) (layer "F.Cu") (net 1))
 (segment (start 140.335 115.09) (end 140.815 115.09) (width 0.3) (layer "F.Cu") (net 1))
 (segment (start 139.965 85.09) (end 140.36 85.485) (width 0.3) (layer "F.Cu") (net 1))
 (segment (start 143.51 106.68) (end 142.72 107.47) (width 0.3) (layer "F.Cu") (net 1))
 (segment (start 133.985 110.04) (end 139.035 115.09) (width 0.3) (layer "F.Cu") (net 1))
 (via (at 128.365 86.9) (size 0.8) (drill 0.4) (layers "F.Cu" "B.Cu") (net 1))
 (via (at 127.825 97.79) (size 0.8) (drill 0.4) (layers "F.Cu" "B.Cu") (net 1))
 (via (at 127.825 92.71) (size 0.8) (drill 0.4) (layers "F.Cu" "B.Cu") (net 1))
 (via (at 127.825 95.25) (size 0.8) (drill 0.4) (layers "F.Cu" "B.Cu") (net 1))
 (via (at 127.825 90.17) (size 0.8) (drill 0.4) (layers "F.Cu" "B.Cu") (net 1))
 (via (at 143.83 92.929002) (size 0.8) (drill 0.4) (layers "F.Cu" "B.Cu") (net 1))
 (via (at 139.51 89.535) (size 0.8) (drill 0.4) (layers "F.Cu" "B.Cu") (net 1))
 (segment (start 128.365 86.9) (end 127.825 87.44) (width 0.3) (layer "B.Cu") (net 1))
 (segment (start 127.825 95.25) (end 127.825 97.79) (width 0.3) (layer "B.Cu") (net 1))
 (segment (start 139.51 91.25) (end 141.189002 92.929002) (width 0.3) (layer "B.Cu") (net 1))
 (segment (start 127.825 92.71) (end 127.825 95.25) (width 0.3) (layer "B.Cu") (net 1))
 (segment (start 139.51 89.535) (end 139.51 91.25) (width 0.3) (layer "B.Cu") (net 1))
 (segment (start 127.825 92.71) (end 127.825 90.17) (width 0.3) (layer "B.Cu") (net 1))
 (segment (start 141.189002 92.929002) (end 143.83 92.929002) (width 0.3) (layer "B.Cu") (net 1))
 (segment (start 127.825 90.17) (end 127.825 87.44) (width 0.3) (layer "B.Cu") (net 1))
 (segment (start 132.281 91.831) (end 132.525 92.075) (width 0.3) (layer "F.Cu") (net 2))
 (segment (start 126.175 90.615) (end 127.391 91.831) (width 0.3) (layer "F.Cu") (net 2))
 (segment (start 127.391 91.831) (end 132.281 91.831) (width 0.3) (layer "F.Cu") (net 2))
 (segment (start 126.175 90.17) (end 119.38 90.17) (width 0.3) (layer "F.Cu") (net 2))
 (segment (start 126.175 90.17) (end 126.175 90.615) (width 0.3) (layer "F.Cu") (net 2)))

